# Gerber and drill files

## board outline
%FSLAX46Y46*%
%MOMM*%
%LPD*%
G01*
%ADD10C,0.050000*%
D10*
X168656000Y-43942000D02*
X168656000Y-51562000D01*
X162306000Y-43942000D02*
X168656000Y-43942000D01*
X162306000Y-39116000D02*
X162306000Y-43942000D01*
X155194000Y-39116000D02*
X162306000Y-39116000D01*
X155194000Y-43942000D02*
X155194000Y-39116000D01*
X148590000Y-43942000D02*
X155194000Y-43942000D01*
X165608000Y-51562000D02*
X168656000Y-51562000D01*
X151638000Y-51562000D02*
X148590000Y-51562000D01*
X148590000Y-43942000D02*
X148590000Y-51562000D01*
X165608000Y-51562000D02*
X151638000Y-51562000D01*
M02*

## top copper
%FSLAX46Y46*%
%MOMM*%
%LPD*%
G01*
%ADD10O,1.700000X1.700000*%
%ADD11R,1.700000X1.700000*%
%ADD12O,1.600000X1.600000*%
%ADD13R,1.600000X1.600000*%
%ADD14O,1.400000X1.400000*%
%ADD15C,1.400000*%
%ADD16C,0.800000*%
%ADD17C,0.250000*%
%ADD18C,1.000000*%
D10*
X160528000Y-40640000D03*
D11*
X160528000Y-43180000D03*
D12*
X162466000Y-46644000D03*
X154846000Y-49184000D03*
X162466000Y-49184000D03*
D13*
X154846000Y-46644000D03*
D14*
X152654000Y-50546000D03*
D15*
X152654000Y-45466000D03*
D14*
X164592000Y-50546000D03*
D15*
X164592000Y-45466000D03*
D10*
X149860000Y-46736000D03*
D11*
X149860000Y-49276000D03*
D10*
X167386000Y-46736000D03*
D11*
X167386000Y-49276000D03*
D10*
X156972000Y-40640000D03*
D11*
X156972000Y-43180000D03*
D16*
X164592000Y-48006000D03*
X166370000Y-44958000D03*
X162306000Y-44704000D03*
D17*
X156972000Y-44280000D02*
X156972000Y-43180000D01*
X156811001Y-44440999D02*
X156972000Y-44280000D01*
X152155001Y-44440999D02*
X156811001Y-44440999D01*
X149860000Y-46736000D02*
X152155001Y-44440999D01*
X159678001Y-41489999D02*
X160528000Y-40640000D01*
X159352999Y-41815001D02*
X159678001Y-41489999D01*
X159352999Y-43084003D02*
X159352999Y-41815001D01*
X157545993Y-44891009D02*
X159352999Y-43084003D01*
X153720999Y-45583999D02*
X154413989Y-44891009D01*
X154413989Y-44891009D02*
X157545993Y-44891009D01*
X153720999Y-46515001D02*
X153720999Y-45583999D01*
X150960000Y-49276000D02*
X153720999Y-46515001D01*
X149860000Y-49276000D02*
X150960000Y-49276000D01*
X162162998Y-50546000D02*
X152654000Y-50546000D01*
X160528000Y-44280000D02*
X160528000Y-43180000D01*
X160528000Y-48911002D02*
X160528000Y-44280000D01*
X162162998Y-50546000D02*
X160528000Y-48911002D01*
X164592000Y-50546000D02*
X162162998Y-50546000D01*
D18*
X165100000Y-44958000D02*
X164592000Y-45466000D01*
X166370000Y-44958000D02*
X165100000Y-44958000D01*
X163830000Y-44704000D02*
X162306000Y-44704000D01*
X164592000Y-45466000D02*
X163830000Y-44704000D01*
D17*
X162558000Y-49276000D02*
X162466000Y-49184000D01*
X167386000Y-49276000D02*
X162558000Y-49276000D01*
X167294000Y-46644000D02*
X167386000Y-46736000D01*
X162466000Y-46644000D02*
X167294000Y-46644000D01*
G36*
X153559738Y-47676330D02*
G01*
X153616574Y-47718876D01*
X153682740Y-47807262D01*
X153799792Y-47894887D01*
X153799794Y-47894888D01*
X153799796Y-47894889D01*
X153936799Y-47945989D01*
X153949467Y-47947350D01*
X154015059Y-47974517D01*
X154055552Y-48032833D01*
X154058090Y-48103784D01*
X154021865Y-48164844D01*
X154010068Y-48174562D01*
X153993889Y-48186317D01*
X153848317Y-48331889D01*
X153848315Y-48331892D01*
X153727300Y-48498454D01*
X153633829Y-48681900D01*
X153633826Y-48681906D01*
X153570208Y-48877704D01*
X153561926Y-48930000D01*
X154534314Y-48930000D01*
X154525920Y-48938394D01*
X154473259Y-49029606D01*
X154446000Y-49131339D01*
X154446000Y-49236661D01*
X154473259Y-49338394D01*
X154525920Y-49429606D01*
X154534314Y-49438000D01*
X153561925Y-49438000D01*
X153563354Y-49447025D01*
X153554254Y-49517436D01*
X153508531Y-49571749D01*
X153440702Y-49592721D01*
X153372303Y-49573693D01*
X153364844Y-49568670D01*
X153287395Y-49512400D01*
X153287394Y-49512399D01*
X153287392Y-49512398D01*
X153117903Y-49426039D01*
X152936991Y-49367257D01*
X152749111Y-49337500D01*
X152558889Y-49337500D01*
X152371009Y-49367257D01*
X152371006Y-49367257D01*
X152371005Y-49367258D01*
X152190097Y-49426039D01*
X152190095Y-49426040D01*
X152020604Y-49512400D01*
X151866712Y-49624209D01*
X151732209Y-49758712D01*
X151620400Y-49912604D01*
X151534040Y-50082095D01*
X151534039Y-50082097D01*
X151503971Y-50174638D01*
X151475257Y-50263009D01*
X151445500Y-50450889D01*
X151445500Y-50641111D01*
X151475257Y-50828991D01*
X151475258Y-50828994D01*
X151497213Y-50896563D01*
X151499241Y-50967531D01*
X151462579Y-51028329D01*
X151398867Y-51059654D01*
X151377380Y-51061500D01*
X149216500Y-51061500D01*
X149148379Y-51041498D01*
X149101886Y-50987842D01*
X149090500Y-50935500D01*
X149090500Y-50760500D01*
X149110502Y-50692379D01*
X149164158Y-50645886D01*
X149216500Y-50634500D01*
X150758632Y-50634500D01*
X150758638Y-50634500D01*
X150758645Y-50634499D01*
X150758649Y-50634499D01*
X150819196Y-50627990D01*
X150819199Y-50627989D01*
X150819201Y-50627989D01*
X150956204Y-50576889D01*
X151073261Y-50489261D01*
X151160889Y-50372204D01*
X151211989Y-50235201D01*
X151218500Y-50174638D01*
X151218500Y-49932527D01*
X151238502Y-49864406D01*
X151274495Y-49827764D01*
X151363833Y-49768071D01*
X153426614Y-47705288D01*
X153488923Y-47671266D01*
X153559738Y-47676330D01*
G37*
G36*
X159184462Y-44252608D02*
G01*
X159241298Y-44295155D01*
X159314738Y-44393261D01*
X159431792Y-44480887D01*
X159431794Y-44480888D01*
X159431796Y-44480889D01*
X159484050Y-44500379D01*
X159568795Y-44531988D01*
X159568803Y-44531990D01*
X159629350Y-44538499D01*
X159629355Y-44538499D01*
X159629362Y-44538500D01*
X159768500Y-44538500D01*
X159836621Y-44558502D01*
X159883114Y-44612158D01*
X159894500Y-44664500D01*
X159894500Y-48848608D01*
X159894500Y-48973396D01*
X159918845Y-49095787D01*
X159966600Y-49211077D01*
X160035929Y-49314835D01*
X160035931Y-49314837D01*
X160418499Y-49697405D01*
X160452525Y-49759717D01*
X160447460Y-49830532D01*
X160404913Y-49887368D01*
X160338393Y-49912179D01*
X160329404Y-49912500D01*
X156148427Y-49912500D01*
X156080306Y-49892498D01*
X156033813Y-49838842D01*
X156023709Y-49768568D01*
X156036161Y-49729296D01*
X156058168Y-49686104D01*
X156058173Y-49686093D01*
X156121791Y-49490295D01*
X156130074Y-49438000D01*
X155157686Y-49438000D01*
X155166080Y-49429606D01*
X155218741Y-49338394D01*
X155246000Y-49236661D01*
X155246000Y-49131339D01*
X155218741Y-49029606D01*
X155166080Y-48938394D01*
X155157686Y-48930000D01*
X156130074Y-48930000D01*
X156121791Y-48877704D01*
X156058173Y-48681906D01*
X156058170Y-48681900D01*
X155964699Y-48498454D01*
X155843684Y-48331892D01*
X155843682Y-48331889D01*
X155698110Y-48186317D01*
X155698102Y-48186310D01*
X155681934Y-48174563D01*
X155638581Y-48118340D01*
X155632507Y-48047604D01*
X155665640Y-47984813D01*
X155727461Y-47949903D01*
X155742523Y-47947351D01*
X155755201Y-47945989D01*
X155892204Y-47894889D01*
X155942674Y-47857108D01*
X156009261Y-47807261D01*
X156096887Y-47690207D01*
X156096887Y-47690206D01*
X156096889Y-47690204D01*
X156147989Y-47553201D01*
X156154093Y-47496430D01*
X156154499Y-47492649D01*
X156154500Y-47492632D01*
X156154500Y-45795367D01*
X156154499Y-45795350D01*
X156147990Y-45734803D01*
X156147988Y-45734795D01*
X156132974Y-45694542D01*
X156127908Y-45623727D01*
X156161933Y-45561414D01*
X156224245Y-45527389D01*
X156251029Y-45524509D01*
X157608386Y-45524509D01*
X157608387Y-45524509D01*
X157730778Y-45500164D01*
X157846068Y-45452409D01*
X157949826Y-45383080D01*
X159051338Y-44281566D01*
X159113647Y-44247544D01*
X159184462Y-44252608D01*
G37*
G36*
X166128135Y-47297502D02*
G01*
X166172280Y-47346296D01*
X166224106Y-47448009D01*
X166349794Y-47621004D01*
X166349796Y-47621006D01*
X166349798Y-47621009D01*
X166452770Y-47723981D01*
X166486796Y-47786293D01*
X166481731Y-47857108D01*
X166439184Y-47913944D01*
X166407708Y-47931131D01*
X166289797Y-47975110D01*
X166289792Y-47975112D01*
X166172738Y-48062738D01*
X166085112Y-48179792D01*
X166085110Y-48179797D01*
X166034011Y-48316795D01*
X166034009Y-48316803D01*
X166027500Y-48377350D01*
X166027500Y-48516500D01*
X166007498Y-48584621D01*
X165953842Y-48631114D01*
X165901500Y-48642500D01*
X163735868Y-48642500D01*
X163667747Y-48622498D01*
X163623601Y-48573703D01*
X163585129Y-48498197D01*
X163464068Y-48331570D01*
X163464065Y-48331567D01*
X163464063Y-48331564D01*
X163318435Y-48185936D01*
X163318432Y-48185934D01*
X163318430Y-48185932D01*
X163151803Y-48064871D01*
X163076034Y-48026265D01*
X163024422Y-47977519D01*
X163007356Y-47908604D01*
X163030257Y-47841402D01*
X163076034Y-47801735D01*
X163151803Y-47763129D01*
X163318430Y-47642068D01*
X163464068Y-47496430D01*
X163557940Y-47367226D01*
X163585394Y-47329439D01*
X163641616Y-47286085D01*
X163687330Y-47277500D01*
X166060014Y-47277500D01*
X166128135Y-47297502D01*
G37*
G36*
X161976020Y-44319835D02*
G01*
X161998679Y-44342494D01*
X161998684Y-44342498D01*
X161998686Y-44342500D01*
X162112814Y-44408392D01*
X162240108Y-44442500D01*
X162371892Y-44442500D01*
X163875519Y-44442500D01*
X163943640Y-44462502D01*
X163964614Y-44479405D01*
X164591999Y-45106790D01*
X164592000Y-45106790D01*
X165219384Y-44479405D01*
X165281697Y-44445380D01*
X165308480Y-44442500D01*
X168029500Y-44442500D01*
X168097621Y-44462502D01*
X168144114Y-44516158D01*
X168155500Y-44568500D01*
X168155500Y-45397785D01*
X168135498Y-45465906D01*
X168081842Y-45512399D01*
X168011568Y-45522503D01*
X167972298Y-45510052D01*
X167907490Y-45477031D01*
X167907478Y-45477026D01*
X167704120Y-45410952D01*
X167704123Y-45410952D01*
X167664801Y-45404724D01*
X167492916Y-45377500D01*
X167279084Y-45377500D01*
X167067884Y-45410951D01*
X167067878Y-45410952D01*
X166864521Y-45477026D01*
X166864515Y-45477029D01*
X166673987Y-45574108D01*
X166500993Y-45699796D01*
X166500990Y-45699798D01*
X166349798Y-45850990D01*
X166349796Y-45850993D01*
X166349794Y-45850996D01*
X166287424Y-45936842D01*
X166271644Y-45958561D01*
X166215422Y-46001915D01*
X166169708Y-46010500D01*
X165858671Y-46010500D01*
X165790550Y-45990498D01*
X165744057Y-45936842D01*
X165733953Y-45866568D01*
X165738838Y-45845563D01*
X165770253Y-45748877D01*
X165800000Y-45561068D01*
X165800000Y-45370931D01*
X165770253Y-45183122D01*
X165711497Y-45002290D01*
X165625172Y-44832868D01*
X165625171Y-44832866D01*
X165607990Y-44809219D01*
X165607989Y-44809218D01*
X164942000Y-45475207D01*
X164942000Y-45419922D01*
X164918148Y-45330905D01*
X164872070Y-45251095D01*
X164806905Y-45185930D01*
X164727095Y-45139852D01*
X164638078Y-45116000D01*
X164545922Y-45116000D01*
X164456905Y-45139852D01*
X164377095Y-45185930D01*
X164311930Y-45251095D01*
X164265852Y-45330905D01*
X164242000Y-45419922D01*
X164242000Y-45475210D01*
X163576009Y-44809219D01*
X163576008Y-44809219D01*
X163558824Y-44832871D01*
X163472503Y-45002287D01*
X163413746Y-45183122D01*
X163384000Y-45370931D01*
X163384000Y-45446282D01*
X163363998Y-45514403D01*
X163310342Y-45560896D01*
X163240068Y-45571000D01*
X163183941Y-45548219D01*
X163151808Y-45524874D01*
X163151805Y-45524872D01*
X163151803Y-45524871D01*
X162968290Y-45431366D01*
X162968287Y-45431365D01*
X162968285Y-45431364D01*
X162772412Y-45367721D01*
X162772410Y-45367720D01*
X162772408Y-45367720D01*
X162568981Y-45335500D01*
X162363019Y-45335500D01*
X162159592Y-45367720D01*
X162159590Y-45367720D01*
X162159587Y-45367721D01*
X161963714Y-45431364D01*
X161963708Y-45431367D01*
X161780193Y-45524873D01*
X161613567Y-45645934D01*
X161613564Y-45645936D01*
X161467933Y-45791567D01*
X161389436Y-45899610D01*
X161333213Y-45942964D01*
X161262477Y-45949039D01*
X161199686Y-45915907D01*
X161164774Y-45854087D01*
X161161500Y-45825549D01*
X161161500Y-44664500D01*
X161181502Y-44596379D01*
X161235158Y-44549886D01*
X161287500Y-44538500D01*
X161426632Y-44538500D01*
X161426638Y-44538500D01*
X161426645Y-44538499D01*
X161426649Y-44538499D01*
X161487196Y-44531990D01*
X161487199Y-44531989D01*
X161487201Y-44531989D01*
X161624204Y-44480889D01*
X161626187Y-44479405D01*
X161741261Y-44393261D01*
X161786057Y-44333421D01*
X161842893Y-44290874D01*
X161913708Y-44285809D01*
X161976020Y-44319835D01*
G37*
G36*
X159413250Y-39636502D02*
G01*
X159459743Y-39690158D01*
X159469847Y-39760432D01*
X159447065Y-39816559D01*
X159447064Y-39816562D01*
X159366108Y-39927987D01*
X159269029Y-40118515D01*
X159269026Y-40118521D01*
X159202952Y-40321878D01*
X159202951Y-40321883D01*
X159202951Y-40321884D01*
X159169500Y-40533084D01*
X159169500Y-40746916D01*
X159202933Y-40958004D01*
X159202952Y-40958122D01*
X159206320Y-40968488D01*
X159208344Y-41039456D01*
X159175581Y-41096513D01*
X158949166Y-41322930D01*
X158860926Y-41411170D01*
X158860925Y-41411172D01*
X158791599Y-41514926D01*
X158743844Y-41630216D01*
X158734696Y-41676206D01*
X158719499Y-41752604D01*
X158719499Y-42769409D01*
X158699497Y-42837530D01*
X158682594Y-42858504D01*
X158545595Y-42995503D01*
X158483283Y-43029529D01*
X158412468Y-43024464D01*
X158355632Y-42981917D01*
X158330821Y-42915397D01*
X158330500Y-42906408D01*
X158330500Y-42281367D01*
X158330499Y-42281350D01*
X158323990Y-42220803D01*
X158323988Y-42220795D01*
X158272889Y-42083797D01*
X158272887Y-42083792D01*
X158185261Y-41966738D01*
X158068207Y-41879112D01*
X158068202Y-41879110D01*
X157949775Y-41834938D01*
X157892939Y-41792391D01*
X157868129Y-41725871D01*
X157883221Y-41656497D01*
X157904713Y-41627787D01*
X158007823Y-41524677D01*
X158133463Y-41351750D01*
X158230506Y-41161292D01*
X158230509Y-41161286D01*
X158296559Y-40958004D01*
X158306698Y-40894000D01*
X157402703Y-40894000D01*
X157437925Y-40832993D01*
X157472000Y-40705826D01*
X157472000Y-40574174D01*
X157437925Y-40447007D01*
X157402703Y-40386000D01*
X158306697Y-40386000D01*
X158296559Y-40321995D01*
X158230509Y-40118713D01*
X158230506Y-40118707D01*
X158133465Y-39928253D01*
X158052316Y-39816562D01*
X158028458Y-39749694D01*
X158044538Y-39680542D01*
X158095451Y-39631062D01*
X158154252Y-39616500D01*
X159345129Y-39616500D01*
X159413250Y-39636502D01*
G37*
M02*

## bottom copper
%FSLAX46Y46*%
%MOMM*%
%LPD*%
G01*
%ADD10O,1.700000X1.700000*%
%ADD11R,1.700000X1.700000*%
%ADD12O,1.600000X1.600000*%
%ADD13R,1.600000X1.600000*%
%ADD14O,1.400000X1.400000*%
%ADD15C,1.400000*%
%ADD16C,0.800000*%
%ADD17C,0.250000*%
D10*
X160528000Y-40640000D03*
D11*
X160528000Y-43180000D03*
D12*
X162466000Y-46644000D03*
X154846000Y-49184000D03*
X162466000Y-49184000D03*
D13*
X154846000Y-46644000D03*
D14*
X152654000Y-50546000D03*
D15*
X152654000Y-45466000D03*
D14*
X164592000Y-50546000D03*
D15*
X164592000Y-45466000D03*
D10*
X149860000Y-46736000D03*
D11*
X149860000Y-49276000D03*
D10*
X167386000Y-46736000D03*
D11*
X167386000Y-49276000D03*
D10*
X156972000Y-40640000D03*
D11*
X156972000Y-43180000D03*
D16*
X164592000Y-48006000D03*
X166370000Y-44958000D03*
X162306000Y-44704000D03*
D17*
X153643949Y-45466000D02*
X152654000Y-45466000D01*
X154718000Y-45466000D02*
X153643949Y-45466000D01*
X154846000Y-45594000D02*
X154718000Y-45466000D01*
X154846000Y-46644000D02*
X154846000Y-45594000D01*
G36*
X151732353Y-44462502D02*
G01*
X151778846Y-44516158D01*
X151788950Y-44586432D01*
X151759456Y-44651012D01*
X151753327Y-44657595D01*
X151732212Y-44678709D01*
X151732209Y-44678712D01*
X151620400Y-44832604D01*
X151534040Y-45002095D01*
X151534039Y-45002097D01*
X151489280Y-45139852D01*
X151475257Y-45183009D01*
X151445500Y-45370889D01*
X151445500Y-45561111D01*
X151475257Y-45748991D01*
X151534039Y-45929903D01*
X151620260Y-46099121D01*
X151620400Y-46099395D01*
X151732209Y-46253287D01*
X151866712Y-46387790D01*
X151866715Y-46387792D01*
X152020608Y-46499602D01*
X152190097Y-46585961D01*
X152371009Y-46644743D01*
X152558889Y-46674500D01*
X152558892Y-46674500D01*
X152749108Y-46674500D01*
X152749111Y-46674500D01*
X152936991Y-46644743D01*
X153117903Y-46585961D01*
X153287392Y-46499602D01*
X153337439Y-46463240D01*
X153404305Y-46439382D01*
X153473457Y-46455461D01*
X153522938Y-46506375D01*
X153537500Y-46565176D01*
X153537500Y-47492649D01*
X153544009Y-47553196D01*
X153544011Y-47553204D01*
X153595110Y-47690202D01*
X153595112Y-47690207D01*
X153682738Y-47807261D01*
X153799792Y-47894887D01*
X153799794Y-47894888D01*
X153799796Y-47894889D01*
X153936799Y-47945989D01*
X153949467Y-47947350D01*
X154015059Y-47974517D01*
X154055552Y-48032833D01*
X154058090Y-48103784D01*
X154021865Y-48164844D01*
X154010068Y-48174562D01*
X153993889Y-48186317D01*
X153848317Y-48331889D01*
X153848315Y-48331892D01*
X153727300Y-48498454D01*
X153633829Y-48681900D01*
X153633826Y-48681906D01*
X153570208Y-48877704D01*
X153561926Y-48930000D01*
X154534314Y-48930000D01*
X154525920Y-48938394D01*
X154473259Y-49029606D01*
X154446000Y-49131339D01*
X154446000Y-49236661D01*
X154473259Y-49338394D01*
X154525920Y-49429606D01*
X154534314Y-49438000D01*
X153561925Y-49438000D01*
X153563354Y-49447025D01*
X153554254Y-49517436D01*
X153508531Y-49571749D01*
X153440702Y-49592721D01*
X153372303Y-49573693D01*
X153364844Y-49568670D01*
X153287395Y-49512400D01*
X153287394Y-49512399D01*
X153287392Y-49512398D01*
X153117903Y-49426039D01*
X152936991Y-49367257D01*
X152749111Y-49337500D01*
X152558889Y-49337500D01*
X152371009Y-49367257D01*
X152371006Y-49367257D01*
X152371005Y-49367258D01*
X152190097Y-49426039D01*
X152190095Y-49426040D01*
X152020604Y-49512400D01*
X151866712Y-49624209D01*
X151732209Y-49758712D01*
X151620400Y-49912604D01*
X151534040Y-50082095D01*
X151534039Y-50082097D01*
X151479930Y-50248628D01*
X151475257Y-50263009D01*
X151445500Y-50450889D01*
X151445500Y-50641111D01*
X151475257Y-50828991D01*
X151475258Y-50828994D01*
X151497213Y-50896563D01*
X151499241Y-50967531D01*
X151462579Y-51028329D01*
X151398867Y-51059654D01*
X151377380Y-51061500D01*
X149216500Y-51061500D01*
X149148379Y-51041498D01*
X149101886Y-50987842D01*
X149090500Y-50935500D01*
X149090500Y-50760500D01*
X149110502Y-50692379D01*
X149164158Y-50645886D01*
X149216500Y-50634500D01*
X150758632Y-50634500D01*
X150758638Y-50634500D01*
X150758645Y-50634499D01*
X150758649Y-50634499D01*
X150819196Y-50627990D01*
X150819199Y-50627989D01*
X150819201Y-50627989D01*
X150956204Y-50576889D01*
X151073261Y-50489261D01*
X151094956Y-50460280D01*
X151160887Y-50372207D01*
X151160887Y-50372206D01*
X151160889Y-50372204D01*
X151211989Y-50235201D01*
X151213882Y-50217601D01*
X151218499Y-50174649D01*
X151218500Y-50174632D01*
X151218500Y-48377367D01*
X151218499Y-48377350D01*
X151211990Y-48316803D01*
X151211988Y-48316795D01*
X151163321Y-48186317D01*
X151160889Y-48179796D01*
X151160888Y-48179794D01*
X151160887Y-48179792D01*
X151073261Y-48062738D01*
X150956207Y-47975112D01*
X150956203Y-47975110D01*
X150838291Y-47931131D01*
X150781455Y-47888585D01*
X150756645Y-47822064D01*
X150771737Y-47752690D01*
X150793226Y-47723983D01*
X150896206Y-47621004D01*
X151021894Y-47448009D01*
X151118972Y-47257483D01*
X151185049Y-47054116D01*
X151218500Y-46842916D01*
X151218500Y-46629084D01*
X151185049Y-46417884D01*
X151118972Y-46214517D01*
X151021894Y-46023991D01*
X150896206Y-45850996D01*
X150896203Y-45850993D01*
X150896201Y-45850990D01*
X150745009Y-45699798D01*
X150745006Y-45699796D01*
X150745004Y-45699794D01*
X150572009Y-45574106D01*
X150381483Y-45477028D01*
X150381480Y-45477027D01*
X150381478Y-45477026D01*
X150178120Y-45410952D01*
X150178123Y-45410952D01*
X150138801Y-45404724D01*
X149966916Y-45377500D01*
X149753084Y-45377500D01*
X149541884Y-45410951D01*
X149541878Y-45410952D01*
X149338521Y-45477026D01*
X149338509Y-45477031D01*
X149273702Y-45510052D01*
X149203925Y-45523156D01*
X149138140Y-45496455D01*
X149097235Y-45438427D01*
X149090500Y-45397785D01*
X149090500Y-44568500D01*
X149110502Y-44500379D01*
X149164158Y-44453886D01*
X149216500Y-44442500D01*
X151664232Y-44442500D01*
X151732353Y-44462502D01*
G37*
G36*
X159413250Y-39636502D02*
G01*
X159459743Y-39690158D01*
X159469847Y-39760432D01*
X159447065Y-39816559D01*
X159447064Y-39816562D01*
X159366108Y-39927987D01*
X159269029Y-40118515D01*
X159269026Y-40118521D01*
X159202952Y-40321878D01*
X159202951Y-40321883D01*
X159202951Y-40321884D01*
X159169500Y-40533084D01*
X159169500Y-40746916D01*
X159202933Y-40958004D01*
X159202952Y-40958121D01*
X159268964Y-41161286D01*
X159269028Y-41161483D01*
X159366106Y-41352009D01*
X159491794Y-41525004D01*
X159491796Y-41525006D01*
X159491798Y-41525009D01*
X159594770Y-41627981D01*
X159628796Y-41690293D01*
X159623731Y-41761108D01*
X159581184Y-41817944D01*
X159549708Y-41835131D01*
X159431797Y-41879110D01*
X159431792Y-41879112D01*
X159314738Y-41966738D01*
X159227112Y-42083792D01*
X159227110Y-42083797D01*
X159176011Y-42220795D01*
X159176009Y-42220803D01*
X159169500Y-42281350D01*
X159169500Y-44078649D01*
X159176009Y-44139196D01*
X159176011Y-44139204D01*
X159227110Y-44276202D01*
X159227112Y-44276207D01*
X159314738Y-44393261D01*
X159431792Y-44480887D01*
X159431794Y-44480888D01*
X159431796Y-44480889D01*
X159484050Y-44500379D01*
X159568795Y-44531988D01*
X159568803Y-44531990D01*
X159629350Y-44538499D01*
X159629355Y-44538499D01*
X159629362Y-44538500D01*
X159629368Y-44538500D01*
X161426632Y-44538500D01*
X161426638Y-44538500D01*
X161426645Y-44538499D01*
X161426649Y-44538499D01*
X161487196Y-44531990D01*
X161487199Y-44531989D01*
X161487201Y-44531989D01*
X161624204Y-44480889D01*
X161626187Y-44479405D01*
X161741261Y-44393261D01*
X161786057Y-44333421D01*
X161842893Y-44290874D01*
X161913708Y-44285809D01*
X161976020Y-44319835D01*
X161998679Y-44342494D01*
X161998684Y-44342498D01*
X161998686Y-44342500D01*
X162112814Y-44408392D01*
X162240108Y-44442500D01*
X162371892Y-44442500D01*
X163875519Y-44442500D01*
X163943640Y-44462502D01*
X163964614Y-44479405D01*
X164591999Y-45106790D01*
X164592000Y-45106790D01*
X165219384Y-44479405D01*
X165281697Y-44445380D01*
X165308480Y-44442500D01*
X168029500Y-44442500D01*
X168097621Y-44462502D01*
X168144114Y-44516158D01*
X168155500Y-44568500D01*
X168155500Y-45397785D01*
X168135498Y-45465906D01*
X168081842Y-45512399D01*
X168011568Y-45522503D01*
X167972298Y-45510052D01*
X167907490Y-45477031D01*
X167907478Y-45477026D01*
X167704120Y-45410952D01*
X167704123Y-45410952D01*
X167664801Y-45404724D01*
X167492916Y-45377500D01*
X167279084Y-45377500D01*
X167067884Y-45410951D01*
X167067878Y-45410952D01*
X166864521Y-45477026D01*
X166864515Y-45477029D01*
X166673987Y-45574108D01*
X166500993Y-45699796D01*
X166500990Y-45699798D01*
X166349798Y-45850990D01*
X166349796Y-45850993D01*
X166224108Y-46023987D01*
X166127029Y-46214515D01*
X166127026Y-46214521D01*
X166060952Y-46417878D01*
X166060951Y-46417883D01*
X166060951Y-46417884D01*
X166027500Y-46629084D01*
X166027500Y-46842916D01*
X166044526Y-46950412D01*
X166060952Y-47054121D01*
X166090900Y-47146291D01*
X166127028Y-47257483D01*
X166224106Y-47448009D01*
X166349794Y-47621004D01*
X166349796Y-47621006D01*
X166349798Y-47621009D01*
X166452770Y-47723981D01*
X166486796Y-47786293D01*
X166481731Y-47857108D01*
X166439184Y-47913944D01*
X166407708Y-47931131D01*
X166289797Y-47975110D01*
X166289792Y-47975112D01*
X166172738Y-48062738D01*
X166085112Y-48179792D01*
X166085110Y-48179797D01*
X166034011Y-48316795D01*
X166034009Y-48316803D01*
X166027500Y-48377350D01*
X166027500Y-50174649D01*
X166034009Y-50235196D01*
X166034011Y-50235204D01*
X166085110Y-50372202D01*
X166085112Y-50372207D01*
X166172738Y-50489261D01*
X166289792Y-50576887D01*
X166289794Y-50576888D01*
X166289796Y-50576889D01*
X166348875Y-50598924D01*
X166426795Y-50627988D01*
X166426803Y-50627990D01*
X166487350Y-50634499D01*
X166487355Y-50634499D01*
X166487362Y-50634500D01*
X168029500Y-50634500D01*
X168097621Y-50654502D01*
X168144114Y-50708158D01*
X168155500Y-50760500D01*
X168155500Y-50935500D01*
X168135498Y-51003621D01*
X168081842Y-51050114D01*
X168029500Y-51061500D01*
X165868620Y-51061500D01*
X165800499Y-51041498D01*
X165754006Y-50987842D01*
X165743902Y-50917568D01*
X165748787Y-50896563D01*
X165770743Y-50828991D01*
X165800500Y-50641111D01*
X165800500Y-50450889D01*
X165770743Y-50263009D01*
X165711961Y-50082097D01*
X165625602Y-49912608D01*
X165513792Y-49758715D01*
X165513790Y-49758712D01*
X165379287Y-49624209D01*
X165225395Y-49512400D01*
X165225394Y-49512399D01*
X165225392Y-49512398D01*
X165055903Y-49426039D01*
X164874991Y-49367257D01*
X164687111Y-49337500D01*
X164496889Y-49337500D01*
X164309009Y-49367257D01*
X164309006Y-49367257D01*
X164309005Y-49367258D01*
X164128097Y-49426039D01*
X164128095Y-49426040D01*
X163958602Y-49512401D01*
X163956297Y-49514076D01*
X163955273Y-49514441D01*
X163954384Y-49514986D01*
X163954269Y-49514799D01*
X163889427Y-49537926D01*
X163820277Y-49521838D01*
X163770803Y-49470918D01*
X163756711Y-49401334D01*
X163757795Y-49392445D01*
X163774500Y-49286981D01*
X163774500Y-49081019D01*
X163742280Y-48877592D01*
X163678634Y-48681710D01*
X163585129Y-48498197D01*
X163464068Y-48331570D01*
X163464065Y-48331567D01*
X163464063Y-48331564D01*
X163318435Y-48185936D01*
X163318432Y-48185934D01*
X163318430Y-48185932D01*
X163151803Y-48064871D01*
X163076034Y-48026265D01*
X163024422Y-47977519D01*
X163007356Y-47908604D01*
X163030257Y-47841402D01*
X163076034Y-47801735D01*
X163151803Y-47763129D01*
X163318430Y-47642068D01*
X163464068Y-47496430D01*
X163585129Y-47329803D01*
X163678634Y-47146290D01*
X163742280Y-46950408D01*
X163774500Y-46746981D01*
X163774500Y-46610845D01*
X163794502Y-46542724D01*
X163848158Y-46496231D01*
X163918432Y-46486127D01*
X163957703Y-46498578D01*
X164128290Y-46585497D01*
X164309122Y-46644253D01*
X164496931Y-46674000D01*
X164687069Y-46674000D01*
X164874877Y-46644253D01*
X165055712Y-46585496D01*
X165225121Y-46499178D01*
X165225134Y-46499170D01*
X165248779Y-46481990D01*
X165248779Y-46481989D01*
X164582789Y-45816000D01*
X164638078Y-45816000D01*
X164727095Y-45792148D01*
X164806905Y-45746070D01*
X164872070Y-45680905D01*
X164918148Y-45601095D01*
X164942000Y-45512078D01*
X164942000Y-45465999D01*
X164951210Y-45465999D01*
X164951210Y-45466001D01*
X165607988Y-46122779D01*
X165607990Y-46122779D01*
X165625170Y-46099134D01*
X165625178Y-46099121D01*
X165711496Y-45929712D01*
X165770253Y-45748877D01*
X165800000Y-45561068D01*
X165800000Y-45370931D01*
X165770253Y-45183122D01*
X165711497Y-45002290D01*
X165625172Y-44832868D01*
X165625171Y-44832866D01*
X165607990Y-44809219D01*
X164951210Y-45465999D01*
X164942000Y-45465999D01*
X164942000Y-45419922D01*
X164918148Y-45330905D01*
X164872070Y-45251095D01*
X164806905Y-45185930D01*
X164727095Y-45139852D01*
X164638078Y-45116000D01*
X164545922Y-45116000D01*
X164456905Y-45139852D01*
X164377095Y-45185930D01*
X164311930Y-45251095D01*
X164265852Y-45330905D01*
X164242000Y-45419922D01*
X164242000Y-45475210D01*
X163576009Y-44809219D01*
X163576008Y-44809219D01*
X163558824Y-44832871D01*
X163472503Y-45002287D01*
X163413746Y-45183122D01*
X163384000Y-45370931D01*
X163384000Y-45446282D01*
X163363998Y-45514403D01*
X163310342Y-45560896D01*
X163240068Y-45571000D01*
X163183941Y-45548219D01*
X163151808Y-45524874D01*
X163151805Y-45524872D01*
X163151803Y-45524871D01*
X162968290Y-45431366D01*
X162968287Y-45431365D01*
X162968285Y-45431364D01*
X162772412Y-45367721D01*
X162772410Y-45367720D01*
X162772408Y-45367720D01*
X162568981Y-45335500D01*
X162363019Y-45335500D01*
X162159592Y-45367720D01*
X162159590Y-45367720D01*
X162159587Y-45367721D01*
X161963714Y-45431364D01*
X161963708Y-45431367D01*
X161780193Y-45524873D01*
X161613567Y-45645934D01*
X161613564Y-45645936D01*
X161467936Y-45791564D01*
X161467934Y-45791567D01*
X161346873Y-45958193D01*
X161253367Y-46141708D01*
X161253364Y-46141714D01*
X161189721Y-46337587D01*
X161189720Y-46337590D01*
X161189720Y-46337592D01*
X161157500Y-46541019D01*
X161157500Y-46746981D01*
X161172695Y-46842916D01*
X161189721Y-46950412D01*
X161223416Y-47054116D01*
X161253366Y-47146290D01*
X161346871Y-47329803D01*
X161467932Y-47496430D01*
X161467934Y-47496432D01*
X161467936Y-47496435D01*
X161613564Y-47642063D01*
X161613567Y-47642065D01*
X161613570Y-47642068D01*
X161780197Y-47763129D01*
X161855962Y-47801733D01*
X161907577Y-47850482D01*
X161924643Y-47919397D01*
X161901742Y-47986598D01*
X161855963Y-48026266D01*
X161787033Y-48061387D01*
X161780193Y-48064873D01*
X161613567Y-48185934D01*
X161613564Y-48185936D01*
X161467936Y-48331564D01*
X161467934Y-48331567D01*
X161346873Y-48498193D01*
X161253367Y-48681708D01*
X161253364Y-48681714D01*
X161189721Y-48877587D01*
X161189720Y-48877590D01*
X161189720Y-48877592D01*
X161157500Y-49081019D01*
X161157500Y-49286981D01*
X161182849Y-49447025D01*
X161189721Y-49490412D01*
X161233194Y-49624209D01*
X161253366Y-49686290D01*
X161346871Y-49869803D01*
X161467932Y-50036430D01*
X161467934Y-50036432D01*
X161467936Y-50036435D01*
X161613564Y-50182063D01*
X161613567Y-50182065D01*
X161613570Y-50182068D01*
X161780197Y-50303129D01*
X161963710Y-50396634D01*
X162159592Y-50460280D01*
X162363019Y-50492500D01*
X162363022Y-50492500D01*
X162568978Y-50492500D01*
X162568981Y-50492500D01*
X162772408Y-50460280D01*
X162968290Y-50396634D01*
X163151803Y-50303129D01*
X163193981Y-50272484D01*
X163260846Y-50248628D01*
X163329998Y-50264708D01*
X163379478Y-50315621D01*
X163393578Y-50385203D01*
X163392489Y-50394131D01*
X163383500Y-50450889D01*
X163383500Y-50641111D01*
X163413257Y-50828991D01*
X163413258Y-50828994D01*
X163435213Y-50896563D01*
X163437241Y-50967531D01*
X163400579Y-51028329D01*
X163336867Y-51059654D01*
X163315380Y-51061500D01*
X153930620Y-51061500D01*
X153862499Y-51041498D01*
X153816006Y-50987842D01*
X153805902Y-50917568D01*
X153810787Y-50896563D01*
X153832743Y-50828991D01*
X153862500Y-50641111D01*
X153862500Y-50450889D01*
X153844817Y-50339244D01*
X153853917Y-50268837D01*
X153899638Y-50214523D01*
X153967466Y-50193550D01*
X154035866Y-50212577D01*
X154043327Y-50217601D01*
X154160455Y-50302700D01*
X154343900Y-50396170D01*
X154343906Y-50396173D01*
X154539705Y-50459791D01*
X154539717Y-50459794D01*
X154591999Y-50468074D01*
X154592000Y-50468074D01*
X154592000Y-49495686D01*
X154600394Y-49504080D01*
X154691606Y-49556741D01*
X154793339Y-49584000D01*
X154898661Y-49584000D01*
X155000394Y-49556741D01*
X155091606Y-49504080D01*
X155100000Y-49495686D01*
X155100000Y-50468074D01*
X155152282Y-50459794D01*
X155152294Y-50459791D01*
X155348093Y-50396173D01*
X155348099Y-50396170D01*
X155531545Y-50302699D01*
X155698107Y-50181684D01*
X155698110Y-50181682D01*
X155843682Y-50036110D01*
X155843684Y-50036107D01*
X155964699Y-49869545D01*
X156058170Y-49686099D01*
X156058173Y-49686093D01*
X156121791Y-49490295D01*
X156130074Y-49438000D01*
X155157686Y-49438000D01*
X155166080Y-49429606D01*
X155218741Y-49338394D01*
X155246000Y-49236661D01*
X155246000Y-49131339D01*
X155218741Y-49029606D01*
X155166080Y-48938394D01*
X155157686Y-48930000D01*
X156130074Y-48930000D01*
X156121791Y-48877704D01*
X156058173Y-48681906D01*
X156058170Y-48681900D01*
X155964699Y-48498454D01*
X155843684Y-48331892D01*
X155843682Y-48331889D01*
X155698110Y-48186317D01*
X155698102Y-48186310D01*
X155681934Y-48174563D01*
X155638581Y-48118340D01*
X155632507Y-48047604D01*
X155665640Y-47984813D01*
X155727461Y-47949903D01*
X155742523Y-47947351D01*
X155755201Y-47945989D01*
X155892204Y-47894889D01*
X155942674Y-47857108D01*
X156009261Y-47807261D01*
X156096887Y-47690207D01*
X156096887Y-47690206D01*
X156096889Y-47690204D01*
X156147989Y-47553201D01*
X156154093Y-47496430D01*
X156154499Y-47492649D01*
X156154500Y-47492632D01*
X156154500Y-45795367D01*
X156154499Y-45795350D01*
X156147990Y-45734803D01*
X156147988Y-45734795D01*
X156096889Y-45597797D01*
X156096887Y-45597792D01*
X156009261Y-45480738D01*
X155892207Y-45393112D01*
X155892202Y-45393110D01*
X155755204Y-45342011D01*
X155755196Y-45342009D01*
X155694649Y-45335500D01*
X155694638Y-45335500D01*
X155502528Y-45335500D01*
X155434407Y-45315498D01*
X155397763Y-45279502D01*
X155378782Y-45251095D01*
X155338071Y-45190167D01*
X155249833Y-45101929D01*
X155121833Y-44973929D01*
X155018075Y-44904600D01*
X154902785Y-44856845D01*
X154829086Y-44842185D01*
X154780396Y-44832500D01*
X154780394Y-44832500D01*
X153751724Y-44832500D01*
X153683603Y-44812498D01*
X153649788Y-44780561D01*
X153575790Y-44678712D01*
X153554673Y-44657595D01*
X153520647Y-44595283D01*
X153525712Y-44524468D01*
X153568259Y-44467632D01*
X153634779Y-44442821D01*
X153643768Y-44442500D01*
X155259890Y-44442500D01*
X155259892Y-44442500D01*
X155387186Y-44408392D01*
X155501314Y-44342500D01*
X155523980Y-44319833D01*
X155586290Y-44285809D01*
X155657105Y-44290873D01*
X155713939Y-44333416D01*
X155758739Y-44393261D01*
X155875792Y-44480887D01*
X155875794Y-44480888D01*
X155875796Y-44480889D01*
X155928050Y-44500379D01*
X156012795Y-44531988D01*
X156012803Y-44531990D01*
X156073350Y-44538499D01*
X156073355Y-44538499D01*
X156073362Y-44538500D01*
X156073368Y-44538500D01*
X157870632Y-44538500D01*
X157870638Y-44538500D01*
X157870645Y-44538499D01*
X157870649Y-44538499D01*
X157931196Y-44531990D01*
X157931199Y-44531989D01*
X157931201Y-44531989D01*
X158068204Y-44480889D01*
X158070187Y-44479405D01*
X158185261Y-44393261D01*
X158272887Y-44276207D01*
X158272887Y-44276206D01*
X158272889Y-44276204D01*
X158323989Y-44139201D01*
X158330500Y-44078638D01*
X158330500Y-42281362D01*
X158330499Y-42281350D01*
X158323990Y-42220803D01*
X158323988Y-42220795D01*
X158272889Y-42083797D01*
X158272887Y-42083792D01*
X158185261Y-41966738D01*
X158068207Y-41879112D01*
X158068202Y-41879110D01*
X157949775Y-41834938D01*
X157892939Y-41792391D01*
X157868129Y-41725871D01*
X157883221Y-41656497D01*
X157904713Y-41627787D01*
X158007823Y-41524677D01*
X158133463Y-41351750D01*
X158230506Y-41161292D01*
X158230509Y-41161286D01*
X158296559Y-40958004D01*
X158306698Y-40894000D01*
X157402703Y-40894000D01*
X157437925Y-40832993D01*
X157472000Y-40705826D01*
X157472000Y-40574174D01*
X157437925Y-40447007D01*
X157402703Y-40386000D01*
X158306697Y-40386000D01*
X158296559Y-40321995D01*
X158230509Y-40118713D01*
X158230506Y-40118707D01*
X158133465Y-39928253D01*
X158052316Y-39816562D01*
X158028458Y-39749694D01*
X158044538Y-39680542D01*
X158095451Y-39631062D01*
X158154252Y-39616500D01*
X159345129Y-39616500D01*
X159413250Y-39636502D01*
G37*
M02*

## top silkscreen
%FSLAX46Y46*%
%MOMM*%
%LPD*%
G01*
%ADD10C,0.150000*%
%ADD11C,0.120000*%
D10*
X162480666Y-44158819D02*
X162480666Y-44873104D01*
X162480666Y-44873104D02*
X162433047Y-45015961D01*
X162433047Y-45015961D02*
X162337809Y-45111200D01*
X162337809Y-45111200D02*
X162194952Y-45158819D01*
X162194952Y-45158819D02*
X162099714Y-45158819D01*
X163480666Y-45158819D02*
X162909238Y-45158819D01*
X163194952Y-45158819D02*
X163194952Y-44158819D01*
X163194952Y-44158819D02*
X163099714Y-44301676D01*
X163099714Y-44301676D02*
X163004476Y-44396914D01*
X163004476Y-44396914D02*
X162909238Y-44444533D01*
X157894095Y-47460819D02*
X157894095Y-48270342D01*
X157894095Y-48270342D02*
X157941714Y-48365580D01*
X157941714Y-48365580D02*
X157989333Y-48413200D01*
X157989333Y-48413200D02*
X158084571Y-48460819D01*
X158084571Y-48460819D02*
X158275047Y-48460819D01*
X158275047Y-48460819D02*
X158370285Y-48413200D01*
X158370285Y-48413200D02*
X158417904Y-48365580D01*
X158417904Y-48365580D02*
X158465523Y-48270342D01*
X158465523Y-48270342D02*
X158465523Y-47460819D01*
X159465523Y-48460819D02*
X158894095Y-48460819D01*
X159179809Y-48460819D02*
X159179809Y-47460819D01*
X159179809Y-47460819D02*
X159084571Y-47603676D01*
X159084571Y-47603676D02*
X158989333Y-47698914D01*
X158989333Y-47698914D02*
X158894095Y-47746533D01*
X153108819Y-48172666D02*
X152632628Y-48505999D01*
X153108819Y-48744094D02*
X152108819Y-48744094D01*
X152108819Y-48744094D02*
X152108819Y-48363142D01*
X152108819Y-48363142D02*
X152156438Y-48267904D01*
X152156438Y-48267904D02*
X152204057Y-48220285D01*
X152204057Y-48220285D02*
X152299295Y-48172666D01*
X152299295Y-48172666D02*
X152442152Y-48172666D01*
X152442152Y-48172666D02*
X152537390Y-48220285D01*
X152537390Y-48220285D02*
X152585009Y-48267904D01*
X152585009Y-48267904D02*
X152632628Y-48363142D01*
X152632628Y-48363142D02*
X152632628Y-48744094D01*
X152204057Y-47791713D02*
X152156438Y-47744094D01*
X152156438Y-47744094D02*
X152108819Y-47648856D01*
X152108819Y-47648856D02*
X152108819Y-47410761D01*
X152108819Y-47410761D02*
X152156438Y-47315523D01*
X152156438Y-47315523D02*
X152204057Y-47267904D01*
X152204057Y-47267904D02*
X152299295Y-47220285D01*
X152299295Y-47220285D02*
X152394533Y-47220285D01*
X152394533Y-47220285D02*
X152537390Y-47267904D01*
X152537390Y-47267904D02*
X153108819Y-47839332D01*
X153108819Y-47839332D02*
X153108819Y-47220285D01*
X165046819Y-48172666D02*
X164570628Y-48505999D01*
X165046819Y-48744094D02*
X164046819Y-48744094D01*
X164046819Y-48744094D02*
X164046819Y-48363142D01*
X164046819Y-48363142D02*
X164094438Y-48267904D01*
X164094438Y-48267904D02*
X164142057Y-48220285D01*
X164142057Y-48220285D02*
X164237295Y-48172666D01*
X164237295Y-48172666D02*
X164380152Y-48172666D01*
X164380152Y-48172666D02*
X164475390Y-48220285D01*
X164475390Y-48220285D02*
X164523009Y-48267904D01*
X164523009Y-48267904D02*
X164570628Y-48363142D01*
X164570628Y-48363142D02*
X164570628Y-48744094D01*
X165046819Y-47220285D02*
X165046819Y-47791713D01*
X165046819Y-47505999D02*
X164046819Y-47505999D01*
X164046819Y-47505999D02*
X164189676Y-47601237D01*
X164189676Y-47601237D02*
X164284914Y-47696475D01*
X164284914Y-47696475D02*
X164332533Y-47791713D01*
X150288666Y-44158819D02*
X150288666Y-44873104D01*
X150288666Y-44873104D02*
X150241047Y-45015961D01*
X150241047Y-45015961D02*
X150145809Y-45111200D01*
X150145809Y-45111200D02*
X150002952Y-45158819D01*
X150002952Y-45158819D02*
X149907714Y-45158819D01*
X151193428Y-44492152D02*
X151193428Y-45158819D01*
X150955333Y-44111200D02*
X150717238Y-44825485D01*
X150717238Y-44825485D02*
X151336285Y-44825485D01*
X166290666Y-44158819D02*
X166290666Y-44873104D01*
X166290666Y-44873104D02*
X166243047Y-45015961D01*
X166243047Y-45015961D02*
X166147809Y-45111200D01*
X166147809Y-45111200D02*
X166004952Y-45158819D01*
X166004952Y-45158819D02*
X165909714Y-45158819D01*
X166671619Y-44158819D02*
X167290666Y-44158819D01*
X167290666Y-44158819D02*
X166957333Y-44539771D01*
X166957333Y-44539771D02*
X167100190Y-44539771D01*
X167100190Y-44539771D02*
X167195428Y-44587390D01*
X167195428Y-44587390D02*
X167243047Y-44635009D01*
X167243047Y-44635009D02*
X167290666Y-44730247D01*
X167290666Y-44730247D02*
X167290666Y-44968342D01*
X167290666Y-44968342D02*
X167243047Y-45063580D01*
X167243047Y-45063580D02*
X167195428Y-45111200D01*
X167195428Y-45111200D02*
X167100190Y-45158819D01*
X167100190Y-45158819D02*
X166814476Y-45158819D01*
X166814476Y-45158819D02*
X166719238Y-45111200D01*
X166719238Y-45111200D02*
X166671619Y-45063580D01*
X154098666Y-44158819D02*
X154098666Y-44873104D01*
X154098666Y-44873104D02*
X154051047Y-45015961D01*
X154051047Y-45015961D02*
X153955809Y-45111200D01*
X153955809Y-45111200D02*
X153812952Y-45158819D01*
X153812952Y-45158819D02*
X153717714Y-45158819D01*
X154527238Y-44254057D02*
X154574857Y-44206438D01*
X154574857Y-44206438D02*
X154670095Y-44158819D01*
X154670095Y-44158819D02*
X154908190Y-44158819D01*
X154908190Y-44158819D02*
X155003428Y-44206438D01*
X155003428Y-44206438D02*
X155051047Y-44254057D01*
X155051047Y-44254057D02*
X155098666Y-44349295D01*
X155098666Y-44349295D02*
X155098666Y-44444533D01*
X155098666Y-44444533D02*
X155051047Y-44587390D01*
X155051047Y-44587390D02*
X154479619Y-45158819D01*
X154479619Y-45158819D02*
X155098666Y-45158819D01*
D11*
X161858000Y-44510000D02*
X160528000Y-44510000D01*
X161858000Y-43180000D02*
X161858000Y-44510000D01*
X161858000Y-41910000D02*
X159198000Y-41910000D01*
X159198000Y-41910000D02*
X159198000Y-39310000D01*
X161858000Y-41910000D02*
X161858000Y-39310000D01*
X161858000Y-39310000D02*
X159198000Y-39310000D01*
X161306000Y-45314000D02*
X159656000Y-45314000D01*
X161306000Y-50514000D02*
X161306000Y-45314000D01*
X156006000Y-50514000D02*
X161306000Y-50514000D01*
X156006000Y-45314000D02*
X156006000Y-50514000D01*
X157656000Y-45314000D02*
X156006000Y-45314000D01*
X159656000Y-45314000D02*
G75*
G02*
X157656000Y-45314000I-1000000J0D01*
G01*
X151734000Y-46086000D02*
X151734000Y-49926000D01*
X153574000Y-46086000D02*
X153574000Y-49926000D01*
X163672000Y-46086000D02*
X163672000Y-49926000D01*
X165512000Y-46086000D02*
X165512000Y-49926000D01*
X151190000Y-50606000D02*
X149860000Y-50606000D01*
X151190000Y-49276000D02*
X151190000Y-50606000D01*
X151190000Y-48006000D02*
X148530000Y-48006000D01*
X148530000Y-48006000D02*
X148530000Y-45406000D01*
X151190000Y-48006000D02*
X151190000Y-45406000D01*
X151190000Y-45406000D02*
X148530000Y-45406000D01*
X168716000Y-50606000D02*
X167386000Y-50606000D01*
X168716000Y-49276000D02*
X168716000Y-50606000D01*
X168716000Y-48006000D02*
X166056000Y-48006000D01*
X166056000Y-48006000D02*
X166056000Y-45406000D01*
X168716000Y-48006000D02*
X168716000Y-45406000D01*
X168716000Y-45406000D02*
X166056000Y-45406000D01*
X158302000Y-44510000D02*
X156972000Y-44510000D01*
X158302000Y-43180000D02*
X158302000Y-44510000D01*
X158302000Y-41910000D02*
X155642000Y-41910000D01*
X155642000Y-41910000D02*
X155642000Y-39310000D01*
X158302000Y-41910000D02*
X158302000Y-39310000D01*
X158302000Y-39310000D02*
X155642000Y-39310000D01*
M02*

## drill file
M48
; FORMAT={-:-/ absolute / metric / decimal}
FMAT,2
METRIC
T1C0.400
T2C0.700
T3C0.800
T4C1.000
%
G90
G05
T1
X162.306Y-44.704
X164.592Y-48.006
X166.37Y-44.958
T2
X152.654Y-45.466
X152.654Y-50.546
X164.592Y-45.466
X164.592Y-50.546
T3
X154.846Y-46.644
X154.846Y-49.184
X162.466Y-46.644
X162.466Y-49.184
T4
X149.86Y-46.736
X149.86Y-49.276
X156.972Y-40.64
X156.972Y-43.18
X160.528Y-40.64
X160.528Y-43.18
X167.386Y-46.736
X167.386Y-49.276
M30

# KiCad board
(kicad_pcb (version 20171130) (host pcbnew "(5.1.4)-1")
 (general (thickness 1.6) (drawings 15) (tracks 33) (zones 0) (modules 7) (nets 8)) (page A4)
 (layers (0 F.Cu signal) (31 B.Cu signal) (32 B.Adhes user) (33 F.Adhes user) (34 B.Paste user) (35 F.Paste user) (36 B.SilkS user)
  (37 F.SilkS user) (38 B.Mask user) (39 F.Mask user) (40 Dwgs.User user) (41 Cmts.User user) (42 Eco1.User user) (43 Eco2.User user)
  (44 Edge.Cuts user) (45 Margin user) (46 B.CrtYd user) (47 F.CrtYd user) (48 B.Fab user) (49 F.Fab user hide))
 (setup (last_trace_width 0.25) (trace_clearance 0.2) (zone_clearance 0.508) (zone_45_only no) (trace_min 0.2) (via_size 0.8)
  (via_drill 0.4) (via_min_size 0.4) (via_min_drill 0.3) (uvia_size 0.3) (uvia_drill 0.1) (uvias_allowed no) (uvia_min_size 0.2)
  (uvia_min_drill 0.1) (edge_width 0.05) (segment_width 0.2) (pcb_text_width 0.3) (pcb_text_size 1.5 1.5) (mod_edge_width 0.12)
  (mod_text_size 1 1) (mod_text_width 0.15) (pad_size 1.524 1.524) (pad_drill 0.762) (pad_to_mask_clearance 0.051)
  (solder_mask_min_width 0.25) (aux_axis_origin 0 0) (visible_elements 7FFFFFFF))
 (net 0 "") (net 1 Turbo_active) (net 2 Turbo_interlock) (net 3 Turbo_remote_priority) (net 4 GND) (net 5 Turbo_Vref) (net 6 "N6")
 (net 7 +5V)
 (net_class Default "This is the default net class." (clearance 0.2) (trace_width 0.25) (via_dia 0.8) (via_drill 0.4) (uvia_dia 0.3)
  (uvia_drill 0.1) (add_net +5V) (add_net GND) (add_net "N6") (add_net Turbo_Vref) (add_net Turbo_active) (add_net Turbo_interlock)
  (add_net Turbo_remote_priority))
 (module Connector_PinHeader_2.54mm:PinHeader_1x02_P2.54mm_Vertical (layer F.Cu) (at 160.528 43.18 180)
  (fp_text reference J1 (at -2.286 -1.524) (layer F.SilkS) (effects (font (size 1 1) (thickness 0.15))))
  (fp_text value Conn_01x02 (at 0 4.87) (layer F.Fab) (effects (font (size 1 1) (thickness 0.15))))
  (fp_line (start -1.33 -1.33) (end 0 -1.33) (layer F.SilkS) (width 0.12))
  (fp_line (start -1.33 0) (end -1.33 -1.33) (layer F.SilkS) (width 0.12))
  (fp_line (start -1.33 1.27) (end 1.33 1.27) (layer F.SilkS) (width 0.12))
  (fp_line (start 1.33 1.27) (end 1.33 3.87) (layer F.SilkS) (width 0.12))
  (fp_line (start -1.33 1.27) (end -1.33 3.87) (layer F.SilkS) (width 0.12))
  (fp_line (start -1.33 3.87) (end 1.33 3.87) (layer F.SilkS) (width 0.12))
  (pad 2 thru_hole oval (at 0 2.54 180) (size 1.7 1.7) (drill 1) (layers *.Cu *.Mask) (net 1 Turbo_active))
  (pad 1 thru_hole rect (at 0 0 180) (size 1.7 1.7) (drill 1) (layers *.Cu *.Mask) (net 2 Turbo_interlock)))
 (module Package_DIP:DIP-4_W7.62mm (layer F.Cu) (at 154.846 46.644)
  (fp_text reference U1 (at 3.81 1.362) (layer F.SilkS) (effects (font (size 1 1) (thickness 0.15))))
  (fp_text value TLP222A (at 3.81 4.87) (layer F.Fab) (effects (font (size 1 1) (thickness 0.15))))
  (fp_line (start 6.46 -1.33) (end 4.81 -1.33) (layer F.SilkS) (width 0.12))
  (fp_line (start 6.46 3.87) (end 6.46 -1.33) (layer F.SilkS) (width 0.12))
  (fp_line (start 1.16 3.87) (end 6.46 3.87) (layer F.SilkS) (width 0.12))
  (fp_line (start 1.16 -1.33) (end 1.16 3.87) (layer F.SilkS) (width 0.12))
  (fp_line (start 2.81 -1.33) (end 1.16 -1.33) (layer F.SilkS) (width 0.12))
  (fp_arc (start 3.81 -1.33) (end 2.81 -1.33) (angle -180) (layer F.SilkS) (width 0.12))
  (pad 4 thru_hole oval (at 7.62 0) (size 1.6 1.6) (drill 0.8) (layers *.Cu *.Mask) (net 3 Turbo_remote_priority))
  (pad 2 thru_hole oval (at 0 2.54) (size 1.6 1.6) (drill 0.8) (layers *.Cu *.Mask) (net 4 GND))
  (pad 3 thru_hole oval (at 7.62 2.54) (size 1.6 1.6) (drill 0.8) (layers *.Cu *.Mask) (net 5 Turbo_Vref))
  (pad 1 thru_hole rect (at 0 0) (size 1.6 1.6) (drill 0.8) (layers *.Cu *.Mask) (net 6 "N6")))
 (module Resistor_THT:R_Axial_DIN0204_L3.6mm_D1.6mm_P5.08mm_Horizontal (layer F.Cu) (at 152.654 45.466 270)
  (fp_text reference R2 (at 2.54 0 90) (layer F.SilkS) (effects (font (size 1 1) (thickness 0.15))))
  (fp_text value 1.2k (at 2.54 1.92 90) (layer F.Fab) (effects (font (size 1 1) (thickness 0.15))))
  (fp_line (start 0.62 0.92) (end 4.46 0.92) (layer F.SilkS) (width 0.12))
  (fp_line (start 0.62 -0.92) (end 4.46 -0.92) (layer F.SilkS) (width 0.12))
  (pad 2 thru_hole oval (at 5.08 0 270) (size 1.4 1.4) (drill 0.7) (layers *.Cu *.Mask) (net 2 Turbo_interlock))
  (pad 1 thru_hole circle (at 0 0 270) (size 1.4 1.4) (drill 0.7) (layers *.Cu *.Mask) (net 6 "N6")))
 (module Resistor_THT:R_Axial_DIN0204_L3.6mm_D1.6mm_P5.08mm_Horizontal (layer F.Cu) (at 164.592 45.466 270)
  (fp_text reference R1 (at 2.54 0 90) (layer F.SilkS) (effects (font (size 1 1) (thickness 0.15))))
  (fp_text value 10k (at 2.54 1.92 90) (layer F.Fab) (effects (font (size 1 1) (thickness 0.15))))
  (fp_line (start 0.62 0.92) (end 4.46 0.92) (layer F.SilkS) (width 0.12))
  (fp_line (start 0.62 -0.92) (end 4.46 -0.92) (layer F.SilkS) (width 0.12))
  (pad 2 thru_hole oval (at 5.08 0 270) (size 1.4 1.4) (drill 0.7) (layers *.Cu *.Mask) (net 2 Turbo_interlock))
  (pad 1 thru_hole circle (at 0 0 270) (size 1.4 1.4) (drill 0.7) (layers *.Cu *.Mask) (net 4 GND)))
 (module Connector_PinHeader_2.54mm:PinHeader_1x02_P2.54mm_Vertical (layer F.Cu) (at 149.86 49.276 180)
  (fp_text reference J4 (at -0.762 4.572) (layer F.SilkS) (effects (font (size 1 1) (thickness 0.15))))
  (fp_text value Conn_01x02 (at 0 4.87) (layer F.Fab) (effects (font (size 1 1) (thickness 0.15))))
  (fp_line (start -1.33 -1.33) (end 0 -1.33) (layer F.SilkS) (width 0.12))
  (fp_line (start -1.33 0) (end -1.33 -1.33) (layer F.SilkS) (width 0.12))
  (fp_line (start -1.33 1.27) (end 1.33 1.27) (layer F.SilkS) (width 0.12))
  (fp_line (start 1.33 1.27) (end 1.33 3.87) (layer F.SilkS) (width 0.12))
  (fp_line (start -1.33 1.27) (end -1.33 3.87) (layer F.SilkS) (width 0.12))
  (fp_line (start -1.33 3.87) (end 1.33 3.87) (layer F.SilkS) (width 0.12))
  (pad 2 thru_hole oval (at 0 2.54 180) (size 1.7 1.7) (drill 1) (layers *.Cu *.Mask) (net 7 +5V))
  (pad 1 thru_hole rect (at 0 0 180) (size 1.7 1.7) (drill 1) (layers *.Cu *.Mask) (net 1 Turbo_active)))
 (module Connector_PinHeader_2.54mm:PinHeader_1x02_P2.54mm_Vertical (layer F.Cu) (at 167.386 49.276 180)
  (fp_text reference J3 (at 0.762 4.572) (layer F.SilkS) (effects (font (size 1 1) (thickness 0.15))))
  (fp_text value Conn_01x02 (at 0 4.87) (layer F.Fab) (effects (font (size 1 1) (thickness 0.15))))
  (fp_line (start -1.33 -1.33) (end 0 -1.33) (layer F.SilkS) (width 0.12))
  (fp_line (start -1.33 0) (end -1.33 -1.33) (layer F.SilkS) (width 0.12))
  (fp_line (start -1.33 1.27) (end 1.33 1.27) (layer F.SilkS) (width 0.12))
  (fp_line (start 1.33 1.27) (end 1.33 3.87) (layer F.SilkS) (width 0.12))
  (fp_line (start -1.33 1.27) (end -1.33 3.87) (layer F.SilkS) (width 0.12))
  (fp_line (start -1.33 3.87) (end 1.33 3.87) (layer F.SilkS) (width 0.12))
  (pad 2 thru_hole oval (at 0 2.54 180) (size 1.7 1.7) (drill 1) (layers *.Cu *.Mask) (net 3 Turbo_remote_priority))
  (pad 1 thru_hole rect (at 0 0 180) (size 1.7 1.7) (drill 1) (layers *.Cu *.Mask) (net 5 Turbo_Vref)))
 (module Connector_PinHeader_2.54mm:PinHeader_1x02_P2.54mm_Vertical (layer F.Cu) (at 156.972 43.18 180)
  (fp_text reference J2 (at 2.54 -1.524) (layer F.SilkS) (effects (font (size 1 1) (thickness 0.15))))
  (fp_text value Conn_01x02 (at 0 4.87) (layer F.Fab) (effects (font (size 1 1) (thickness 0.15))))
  (fp_line (start -1.33 -1.33) (end 0 -1.33) (layer F.SilkS) (width 0.12))
  (fp_line (start -1.33 0) (end -1.33 -1.33) (layer F.SilkS) (width 0.12))
  (fp_line (start -1.33 1.27) (end 1.33 1.27) (layer F.SilkS) (width 0.12))
  (fp_line (start 1.33 1.27) (end 1.33 3.87) (layer F.SilkS) (width 0.12))
  (fp_line (start -1.33 1.27) (end -1.33 3.87) (layer F.SilkS) (width 0.12))
  (fp_line (start -1.33 3.87) (end 1.33 3.87) (layer F.SilkS) (width 0.12))
  (pad 2 thru_hole oval (at 0 2.54 180) (size 1.7 1.7) (drill 1) (layers *.Cu *.Mask) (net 4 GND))
  (pad 1 thru_hole rect (at 0 0 180) (size 1.7 1.7) (drill 1) (layers *.Cu *.Mask) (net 7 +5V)))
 (gr_line (start 168.656 43.942) (end 168.656 51.562) (layer Edge.Cuts) (width 0.05))
 (gr_line (start 162.306 43.942) (end 168.656 43.942) (layer Edge.Cuts) (width 0.05))
 (gr_line (start 162.306 39.116) (end 162.306 43.942) (layer Edge.Cuts) (width 0.05))
 (gr_line (start 155.194 39.116) (end 162.306 39.116) (layer Edge.Cuts) (width 0.05))
 (gr_line (start 155.194 43.942) (end 155.194 39.116) (layer Edge.Cuts) (width 0.05))
 (gr_line (start 148.59 43.942) (end 155.194 43.942) (layer Edge.Cuts) (width 0.05))
 (gr_line (start 165.608 51.562) (end 168.656 51.562) (layer Edge.Cuts) (width 0.05))
 (gr_line (start 151.638 51.562) (end 148.59 51.562) (layer Edge.Cuts) (width 0.05))
 (gr_line (start 148.59 43.942) (end 148.59 51.562) (layer Edge.Cuts) (width 0.05))
 (gr_line (start 165.608 51.562) (end 151.638 51.562) (layer Edge.Cuts) (width 0.05))
 (segment (start 156.972 44.28) (end 156.972 43.18) (width 0.25) (layer F.Cu) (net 7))
 (segment (start 156.811001 44.440999) (end 156.972 44.28) (width 0.25) (layer F.Cu) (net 7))
 (segment (start 152.155001 44.440999) (end 156.811001 44.440999) (width 0.25) (layer F.Cu) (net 7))
 (segment (start 149.86 46.736) (end 152.155001 44.440999) (width 0.25) (layer F.Cu) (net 7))
 (segment (start 159.678001 41.489999) (end 160.528 40.64) (width 0.25) (layer F.Cu) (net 1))
 (segment (start 159.352999 41.815001) (end 159.678001 41.489999) (width 0.25) (layer F.Cu) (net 1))
 (segment (start 159.352999 43.084003) (end 159.352999 41.815001) (width 0.25) (layer F.Cu) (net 1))
 (segment (start 157.545993 44.891009) (end 159.352999 43.084003) (width 0.25) (layer F.Cu) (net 1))
 (segment (start 153.720999 45.583999) (end 154.413989 44.891009) (width 0.25) (layer F.Cu) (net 1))
 (segment (start 154.413989 44.891009) (end 157.545993 44.891009) (width 0.25) (layer F.Cu) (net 1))
 (segment (start 153.720999 46.515001) (end 153.720999 45.583999) (width 0.25) (layer F.Cu) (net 1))
 (segment (start 150.96 49.276) (end 153.720999 46.515001) (width 0.25) (layer F.Cu) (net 1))
 (segment (start 149.86 49.276) (end 150.96 49.276) (width 0.25) (layer F.Cu) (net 1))
 (segment (start 162.162998 50.546) (end 152.654 50.546) (width 0.25) (layer F.Cu) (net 2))
 (segment (start 160.528 44.28) (end 160.528 43.18) (width 0.25) (layer F.Cu) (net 2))
 (segment (start 160.528 48.911002) (end 160.528 44.28) (width 0.25) (layer F.Cu) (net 2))
 (segment (start 162.162998 50.546) (end 160.528 48.911002) (width 0.25) (layer F.Cu) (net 2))
 (segment (start 164.592 50.546) (end 162.162998 50.546) (width 0.25) (layer F.Cu) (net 2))
 (via (at 164.592 48.006) (size 0.8) (drill 0.4) (layers F.Cu B.Cu) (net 4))
 (via (at 166.37 44.958) (size 0.8) (drill 0.4) (layers F.Cu B.Cu) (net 4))
 (via (at 162.306 44.704) (size 0.8) (drill 0.4) (layers F.Cu B.Cu) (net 4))
 (segment (start 165.1 44.958) (end 164.592 45.466) (width 1) (layer F.Cu) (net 4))
 (segment (start 166.37 44.958) (end 165.1 44.958) (width 1) (layer F.Cu) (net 4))
 (segment (start 163.83 44.704) (end 162.306 44.704) (width 1) (layer F.Cu) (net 4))
 (segment (start 164.592 45.466) (end 163.83 44.704) (width 1) (layer F.Cu) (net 4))
 (segment (start 162.558 49.276) (end 162.466 49.184) (width 0.25) (layer F.Cu) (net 5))
 (segment (start 167.386 49.276) (end 162.558 49.276) (width 0.25) (layer F.Cu) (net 5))
 (segment (start 153.643949 45.466) (end 152.654 45.466) (width 0.25) (layer B.Cu) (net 6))
 (segment (start 154.718 45.466) (end 153.643949 45.466) (width 0.25) (layer B.Cu) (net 6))
 (segment (start 154.846 45.594) (end 154.718 45.466) (width 0.25) (layer B.Cu) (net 6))
 (segment (start 154.846 46.644) (end 154.846 45.594) (width 0.25) (layer B.Cu) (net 6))
 (segment (start 167.294 46.644) (end 167.386 46.736) (width 0.25) (layer F.Cu) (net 3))
 (segment (start 162.466 46.644) (end 167.294 46.644) (width 0.25) (layer F.Cu) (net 3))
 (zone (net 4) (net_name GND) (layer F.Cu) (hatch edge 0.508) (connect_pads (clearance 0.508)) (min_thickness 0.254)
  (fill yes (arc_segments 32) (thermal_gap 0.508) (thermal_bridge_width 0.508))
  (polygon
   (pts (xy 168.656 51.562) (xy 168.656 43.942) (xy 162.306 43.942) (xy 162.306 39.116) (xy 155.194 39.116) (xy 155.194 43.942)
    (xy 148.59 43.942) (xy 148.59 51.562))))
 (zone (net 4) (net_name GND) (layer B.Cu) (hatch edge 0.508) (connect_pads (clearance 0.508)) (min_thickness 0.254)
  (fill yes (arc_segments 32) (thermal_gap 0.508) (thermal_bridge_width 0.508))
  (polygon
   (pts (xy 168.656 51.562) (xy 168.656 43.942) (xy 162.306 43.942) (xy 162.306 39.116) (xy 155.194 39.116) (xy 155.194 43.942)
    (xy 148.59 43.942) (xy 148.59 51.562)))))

